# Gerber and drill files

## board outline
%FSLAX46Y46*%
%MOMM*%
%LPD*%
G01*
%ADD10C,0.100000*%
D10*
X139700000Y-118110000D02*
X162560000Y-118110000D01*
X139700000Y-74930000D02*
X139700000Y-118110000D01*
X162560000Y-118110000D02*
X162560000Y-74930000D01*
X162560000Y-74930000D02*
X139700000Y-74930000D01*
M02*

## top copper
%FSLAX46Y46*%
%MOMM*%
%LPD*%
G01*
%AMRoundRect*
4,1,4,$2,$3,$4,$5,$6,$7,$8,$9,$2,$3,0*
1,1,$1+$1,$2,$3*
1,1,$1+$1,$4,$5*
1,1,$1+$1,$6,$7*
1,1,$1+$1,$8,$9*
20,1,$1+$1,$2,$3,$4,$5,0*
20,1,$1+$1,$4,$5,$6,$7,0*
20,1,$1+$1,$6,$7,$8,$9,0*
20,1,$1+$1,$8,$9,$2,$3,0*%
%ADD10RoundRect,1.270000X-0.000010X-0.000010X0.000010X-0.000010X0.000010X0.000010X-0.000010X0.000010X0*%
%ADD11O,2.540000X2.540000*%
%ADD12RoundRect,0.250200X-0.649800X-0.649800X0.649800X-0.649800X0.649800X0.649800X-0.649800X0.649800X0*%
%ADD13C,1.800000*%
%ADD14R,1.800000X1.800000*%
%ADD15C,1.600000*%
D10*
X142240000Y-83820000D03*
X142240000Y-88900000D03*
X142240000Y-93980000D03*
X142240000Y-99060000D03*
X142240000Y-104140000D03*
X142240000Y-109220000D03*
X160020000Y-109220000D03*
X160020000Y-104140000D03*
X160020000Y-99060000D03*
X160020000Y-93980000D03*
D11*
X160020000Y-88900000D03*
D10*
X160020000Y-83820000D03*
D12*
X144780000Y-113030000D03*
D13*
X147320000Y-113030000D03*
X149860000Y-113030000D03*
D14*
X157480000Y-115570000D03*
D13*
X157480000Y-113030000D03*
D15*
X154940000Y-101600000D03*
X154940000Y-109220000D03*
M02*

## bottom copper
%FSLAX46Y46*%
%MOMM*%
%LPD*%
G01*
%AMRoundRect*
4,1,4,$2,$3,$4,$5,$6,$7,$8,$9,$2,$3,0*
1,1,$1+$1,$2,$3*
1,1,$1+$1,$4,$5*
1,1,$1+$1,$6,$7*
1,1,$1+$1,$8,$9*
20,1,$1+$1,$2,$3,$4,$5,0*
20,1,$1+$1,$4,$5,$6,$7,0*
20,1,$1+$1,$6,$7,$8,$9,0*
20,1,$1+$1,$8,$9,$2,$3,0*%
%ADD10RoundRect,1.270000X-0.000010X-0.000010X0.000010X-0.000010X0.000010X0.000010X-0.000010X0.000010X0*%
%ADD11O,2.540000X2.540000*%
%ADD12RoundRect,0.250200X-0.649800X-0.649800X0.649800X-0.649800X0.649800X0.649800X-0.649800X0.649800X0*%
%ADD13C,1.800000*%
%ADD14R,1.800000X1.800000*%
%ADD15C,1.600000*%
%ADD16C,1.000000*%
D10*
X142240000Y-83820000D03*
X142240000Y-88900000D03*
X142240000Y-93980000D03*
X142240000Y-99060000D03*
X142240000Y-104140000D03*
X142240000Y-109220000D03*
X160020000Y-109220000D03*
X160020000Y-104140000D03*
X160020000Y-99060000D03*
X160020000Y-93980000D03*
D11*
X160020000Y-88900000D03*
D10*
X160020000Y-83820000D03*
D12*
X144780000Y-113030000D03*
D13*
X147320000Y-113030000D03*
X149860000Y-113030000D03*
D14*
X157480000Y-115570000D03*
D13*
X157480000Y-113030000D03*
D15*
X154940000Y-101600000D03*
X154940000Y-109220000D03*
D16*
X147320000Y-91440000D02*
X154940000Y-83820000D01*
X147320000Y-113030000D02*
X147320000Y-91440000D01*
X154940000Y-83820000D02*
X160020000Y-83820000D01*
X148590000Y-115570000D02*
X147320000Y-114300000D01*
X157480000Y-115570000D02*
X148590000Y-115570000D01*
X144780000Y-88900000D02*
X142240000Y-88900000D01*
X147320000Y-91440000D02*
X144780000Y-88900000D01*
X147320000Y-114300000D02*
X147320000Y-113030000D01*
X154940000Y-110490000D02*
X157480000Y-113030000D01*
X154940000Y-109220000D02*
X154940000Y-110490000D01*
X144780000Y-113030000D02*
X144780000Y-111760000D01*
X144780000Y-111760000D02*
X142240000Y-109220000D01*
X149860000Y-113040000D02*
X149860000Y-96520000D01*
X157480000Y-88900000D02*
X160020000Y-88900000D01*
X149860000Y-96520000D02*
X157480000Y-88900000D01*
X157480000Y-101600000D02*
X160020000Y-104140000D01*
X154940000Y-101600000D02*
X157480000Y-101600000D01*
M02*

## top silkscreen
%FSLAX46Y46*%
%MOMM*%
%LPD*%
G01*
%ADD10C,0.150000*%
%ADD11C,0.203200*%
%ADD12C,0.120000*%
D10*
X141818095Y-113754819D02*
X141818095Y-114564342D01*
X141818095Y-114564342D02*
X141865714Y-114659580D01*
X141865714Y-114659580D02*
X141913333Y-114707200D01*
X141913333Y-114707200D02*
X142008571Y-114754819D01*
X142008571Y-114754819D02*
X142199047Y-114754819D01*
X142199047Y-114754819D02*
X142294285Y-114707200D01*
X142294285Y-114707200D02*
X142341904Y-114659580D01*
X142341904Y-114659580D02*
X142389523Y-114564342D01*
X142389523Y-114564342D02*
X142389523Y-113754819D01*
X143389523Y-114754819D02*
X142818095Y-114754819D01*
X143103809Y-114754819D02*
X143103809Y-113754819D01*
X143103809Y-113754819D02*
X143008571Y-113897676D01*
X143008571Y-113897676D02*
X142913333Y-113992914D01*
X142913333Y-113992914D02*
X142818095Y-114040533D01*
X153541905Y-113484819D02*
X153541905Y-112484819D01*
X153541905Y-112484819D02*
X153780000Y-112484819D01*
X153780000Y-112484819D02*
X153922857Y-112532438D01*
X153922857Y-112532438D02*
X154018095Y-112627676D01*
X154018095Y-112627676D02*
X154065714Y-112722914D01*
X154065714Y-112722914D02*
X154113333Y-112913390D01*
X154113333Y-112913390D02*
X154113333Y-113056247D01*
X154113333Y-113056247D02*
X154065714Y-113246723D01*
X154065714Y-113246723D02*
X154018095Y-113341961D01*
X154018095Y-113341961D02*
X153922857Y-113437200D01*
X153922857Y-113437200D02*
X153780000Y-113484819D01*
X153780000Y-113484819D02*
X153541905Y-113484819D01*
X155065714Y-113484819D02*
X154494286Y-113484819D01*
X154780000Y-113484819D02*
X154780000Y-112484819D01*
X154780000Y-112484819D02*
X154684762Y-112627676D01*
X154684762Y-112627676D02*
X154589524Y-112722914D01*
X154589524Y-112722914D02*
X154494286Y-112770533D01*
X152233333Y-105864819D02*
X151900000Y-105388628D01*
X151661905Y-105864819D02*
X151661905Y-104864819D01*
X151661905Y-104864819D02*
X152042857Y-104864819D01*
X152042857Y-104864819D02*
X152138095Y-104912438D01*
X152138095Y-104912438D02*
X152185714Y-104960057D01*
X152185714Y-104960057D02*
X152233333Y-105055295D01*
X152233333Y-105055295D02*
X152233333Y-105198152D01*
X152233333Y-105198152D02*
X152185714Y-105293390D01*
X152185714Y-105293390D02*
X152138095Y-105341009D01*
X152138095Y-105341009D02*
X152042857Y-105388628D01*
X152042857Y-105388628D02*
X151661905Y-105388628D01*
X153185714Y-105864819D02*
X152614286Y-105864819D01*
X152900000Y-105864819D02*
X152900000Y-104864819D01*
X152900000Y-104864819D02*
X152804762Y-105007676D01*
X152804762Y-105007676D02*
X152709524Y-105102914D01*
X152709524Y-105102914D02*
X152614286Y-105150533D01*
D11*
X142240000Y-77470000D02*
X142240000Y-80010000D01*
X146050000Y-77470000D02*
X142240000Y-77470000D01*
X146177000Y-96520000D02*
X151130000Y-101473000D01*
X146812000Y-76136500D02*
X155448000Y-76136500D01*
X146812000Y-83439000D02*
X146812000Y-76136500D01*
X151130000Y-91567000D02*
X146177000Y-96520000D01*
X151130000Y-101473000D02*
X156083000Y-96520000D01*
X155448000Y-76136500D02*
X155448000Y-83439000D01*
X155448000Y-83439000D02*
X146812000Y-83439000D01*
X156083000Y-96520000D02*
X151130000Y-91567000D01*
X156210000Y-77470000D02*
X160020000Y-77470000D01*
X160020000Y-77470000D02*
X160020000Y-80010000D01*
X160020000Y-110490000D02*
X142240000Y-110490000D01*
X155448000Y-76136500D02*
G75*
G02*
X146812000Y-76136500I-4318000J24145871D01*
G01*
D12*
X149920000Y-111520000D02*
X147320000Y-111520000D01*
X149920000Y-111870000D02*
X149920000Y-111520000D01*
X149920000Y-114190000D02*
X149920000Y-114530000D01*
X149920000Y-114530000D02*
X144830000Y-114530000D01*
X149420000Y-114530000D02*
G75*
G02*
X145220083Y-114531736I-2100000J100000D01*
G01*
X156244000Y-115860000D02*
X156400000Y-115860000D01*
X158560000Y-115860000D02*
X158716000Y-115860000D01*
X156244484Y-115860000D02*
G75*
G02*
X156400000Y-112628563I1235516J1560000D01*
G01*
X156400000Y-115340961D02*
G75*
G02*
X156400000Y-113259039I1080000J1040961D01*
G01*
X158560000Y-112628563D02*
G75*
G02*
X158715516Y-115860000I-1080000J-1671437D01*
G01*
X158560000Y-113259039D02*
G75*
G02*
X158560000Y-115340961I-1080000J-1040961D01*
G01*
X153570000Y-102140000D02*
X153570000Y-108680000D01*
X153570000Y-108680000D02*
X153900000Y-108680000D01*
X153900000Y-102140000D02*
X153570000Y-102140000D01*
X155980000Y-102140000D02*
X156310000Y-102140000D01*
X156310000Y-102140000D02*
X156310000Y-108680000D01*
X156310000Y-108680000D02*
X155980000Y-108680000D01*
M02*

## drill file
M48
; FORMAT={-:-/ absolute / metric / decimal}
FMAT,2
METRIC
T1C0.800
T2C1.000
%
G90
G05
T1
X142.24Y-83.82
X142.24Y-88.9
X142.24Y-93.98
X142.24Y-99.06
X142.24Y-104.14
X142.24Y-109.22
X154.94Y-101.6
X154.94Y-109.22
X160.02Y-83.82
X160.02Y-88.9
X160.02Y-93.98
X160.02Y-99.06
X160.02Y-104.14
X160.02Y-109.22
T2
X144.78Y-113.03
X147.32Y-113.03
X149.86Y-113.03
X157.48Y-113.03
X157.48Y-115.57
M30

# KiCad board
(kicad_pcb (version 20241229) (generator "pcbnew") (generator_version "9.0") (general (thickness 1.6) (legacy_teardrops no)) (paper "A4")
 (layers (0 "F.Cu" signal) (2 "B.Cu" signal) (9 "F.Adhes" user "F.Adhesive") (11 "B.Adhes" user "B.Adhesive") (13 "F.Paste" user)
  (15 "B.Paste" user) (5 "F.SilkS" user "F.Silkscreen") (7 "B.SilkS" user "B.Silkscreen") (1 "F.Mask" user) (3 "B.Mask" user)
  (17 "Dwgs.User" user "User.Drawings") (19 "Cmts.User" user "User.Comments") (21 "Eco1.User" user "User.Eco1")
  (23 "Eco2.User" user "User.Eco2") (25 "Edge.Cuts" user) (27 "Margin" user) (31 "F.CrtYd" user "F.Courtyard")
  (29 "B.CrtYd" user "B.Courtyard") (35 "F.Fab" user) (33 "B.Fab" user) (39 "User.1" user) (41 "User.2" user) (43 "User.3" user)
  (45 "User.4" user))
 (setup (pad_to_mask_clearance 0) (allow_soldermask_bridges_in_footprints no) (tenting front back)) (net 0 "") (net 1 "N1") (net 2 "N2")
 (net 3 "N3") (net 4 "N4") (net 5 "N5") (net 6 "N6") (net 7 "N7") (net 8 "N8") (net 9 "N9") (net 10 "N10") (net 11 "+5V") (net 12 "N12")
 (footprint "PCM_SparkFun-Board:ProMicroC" (layer "F.Cu") (at 151.13 93.98)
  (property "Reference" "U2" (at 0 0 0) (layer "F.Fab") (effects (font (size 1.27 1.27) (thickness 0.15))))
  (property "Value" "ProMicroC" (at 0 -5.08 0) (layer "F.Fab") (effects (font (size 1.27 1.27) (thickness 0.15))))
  (fp_line (start -8.89 -16.51) (end -8.89 -13.97) (stroke (width 0.2032) (type solid)) (layer "F.SilkS"))
  (fp_line (start -5.08 -16.51) (end -8.89 -16.51) (stroke (width 0.2032) (type solid)) (layer "F.SilkS"))
  (fp_line (start -4.953 2.54) (end 0 7.493) (stroke (width 0.2032) (type solid)) (layer "F.SilkS"))
  (fp_line (start -4.318 -17.8435) (end 4.318 -17.8435) (stroke (width 0.2032) (type solid)) (layer "F.SilkS"))
  (fp_line (start -4.318 -10.541) (end -4.318 -17.8435) (stroke (width 0.2032) (type solid)) (layer "F.SilkS"))
  (fp_line (start 0 -2.413) (end -4.953 2.54) (stroke (width 0.2032) (type solid)) (layer "F.SilkS"))
  (fp_line (start 0 7.493) (end 4.953 2.54) (stroke (width 0.2032) (type solid)) (layer "F.SilkS"))
  (fp_line (start 4.318 -17.8435) (end 4.318 -10.541) (stroke (width 0.2032) (type solid)) (layer "F.SilkS"))
  (fp_line (start 4.318 -10.541) (end -4.318 -10.541) (stroke (width 0.2032) (type solid)) (layer "F.SilkS"))
  (fp_line (start 4.953 2.54) (end 0 -2.413) (stroke (width 0.2032) (type solid)) (layer "F.SilkS"))
  (fp_line (start 5.08 -16.51) (end 8.89 -16.51) (stroke (width 0.2032) (type solid)) (layer "F.SilkS"))
  (fp_line (start 8.89 -16.51) (end 8.89 -13.97) (stroke (width 0.2032) (type solid)) (layer "F.SilkS"))
  (fp_line (start 8.89 16.51) (end -8.89 16.51) (stroke (width 0.2032) (type solid)) (layer "F.SilkS"))
  (fp_arc (start 4.318 -17.8435) (mid 0 -17.460445) (end -4.318 -17.8435) (stroke (width 0.2032) (type solid)) (layer "F.SilkS"))
  (pad "2" thru_hole roundrect (at -8.89 -10.16) (size 2.54 2.54) (drill 0.8) (layers "*.Cu" "*.Mask") (remove_unused_layers no)
   (roundrect_rratio 0.5) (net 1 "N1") (thermal_bridge_angle 0))
  (pad "4" thru_hole roundrect (at -8.89 -5.08) (size 2.54 2.54) (drill 0.8) (layers "*.Cu" "*.Mask") (remove_unused_layers no)
   (roundrect_rratio 0.5) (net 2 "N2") (thermal_bridge_angle 0))
  (pad "6" thru_hole roundrect (at -8.89 0) (size 2.54 2.54) (drill 0.8) (layers "*.Cu" "*.Mask") (remove_unused_layers no)
   (roundrect_rratio 0.5) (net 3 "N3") (thermal_bridge_angle 0))
  (pad "8" thru_hole roundrect (at -8.89 5.08) (size 2.54 2.54) (drill 0.8) (layers "*.Cu" "*.Mask") (remove_unused_layers no)
   (roundrect_rratio 0.5) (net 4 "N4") (thermal_bridge_angle 0))
  (pad "10" thru_hole roundrect (at -8.89 10.16) (size 2.54 2.54) (drill 0.8) (layers "*.Cu" "*.Mask") (remove_unused_layers no)
   (roundrect_rratio 0.5) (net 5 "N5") (thermal_bridge_angle 0))
  (pad "12" thru_hole roundrect (at -8.89 15.24) (size 2.54 2.54) (drill 0.8) (layers "*.Cu" "*.Mask") (remove_unused_layers no)
   (roundrect_rratio 0.5) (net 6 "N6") (thermal_bridge_angle 0))
  (pad "13" thru_hole roundrect (at 8.89 15.24) (size 2.54 2.54) (drill 0.8) (layers "*.Cu" "*.Mask") (remove_unused_layers no)
   (roundrect_rratio 0.5) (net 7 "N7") (thermal_bridge_angle 0))
  (pad "15" thru_hole roundrect (at 8.89 10.16) (size 2.54 2.54) (drill 0.8) (layers "*.Cu" "*.Mask") (remove_unused_layers no)
   (roundrect_rratio 0.5) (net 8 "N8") (thermal_bridge_angle 0))
  (pad "17" thru_hole roundrect (at 8.89 5.08) (size 2.54 2.54) (drill 0.8) (layers "*.Cu" "*.Mask") (remove_unused_layers no)
   (roundrect_rratio 0.5) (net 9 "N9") (thermal_bridge_angle 0))
  (pad "19" thru_hole roundrect (at 8.89 0) (size 2.54 2.54) (drill 0.8) (layers "*.Cu" "*.Mask") (remove_unused_layers no)
   (roundrect_rratio 0.5) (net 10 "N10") (thermal_bridge_angle 0))
  (pad "21" thru_hole oval (at 8.89 -5.08) (size 2.54 2.54) (drill 0.8) (layers "*.Cu" "*.Mask") (remove_unused_layers no) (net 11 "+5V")
   (thermal_bridge_angle 0))
  (pad "23" thru_hole roundrect (at 8.89 -10.16) (size 2.54 2.54) (drill 0.8) (layers "*.Cu" "*.Mask") (remove_unused_layers no)
   (roundrect_rratio 0.5) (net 2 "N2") (thermal_bridge_angle 0)))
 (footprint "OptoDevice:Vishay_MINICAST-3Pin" (layer "F.Cu") (at 144.78 113.03)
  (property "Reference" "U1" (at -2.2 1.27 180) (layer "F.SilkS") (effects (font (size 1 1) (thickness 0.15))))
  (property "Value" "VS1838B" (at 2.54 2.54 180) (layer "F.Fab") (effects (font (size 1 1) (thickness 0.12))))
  (fp_line (start 5.14 -1.51) (end 2.54 -1.51) (stroke (width 0.12) (type solid)) (layer "F.SilkS"))
  (fp_line (start 5.14 -1.16) (end 5.14 -1.51) (stroke (width 0.12) (type solid)) (layer "F.SilkS"))
  (fp_line (start 5.14 1.16) (end 5.14 1.5) (stroke (width 0.12) (type solid)) (layer "F.SilkS"))
  (fp_line (start 5.14 1.5) (end 0.05 1.5) (stroke (width 0.12) (type solid)) (layer "F.SilkS"))
  (fp_arc (start 4.64 1.5) (mid 2.540869 3.502379) (end 0.440083 1.501736) (stroke (width 0.12) (type solid)) (layer "F.SilkS"))
  (pad "1" thru_hole roundrect (at 0 0) (size 1.8 1.8) (drill 1) (layers "*.Cu" "*.Mask") (remove_unused_layers no) (roundrect_rratio 0.139)
   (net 6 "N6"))
  (pad "2" thru_hole circle (at 2.54 0) (size 1.8 1.8) (drill 1) (layers "*.Cu" "*.Mask") (remove_unused_layers no) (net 2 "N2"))
  (pad "3" thru_hole circle (at 5.08 0) (size 1.8 1.8) (drill 1) (layers "*.Cu" "*.Mask") (remove_unused_layers no) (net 11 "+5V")))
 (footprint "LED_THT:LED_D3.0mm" (layer "F.Cu") (at 157.48 115.57 90)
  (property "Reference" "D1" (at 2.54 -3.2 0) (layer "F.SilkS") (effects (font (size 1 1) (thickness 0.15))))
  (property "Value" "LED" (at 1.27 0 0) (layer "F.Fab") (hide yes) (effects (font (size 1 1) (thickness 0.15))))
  (fp_line (start -0.29 -1.236) (end -0.29 -1.08) (stroke (width 0.12) (type solid)) (layer "F.SilkS"))
  (fp_line (start -0.29 1.08) (end -0.29 1.236) (stroke (width 0.12) (type solid)) (layer "F.SilkS"))
  (fp_arc (start -0.29 -1.235516) (mid 1.36566 -1.987699) (end 2.941437 -1.08) (stroke (width 0.12) (type solid)) (layer "F.SilkS"))
  (fp_arc (start 0.229039 -1.08) (mid 1.27 -1.5) (end 2.310961 -1.08) (stroke (width 0.12) (type solid)) (layer "F.SilkS"))
  (fp_arc (start 2.941437 1.08) (mid 1.36566 1.987699) (end -0.29 1.235516) (stroke (width 0.12) (type solid)) (layer "F.SilkS"))
  (fp_arc (start 2.310961 1.08) (mid 1.27 1.5) (end 0.229039 1.08) (stroke (width 0.12) (type solid)) (layer "F.SilkS"))
  (pad "1" thru_hole rect (at 0 0 90) (size 1.8 1.8) (drill 1) (layers "*.Cu" "*.Mask") (remove_unused_layers no) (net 2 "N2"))
  (pad "2" thru_hole circle (at 2.54 0 90) (size 1.8 1.8) (drill 1) (layers "*.Cu" "*.Mask") (remove_unused_layers no) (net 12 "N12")))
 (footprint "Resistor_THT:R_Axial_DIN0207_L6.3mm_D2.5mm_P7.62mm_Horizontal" (layer "F.Cu") (at 154.94 101.6 -90)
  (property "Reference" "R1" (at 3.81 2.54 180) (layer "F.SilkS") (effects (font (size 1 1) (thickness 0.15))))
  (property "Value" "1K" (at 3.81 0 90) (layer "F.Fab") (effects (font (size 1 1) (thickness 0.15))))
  (fp_line (start 0.54 1.37) (end 7.08 1.37) (stroke (width 0.12) (type solid)) (layer "F.SilkS"))
  (fp_line (start 7.08 1.37) (end 7.08 1.04) (stroke (width 0.12) (type solid)) (layer "F.SilkS"))
  (fp_line (start 0.54 1.04) (end 0.54 1.37) (stroke (width 0.12) (type solid)) (layer "F.SilkS"))
  (fp_line (start 0.54 -1.04) (end 0.54 -1.37) (stroke (width 0.12) (type solid)) (layer "F.SilkS"))
  (fp_line (start 0.54 -1.37) (end 7.08 -1.37) (stroke (width 0.12) (type solid)) (layer "F.SilkS"))
  (fp_line (start 7.08 -1.37) (end 7.08 -1.04) (stroke (width 0.12) (type solid)) (layer "F.SilkS"))
  (pad "1" thru_hole circle (at 0 0 270) (size 1.6 1.6) (drill 0.8) (layers "*.Cu" "*.Mask") (remove_unused_layers no) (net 8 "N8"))
  (pad "2" thru_hole circle (at 7.62 0 270) (size 1.6 1.6) (drill 0.8) (layers "*.Cu" "*.Mask") (remove_unused_layers no) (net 12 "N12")))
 (gr_line (start 139.7 118.11) (end 162.56 118.11) (stroke (width 0.1) (type solid)) (layer "Edge.Cuts"))
 (gr_line (start 139.7 74.93) (end 139.7 118.11) (stroke (width 0.1) (type default)) (layer "Edge.Cuts"))
 (gr_line (start 162.56 118.11) (end 162.56 74.93) (stroke (width 0.1) (type default)) (layer "Edge.Cuts"))
 (gr_line (start 162.56 74.93) (end 139.7 74.93) (stroke (width 0.1) (type solid)) (layer "Edge.Cuts"))
 (segment (start 147.32 91.44) (end 154.94 83.82) (width 1) (layer "B.Cu") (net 2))
 (segment (start 147.32 113.03) (end 147.32 91.44) (width 1) (layer "B.Cu") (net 2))
 (segment (start 154.94 83.82) (end 160.02 83.82) (width 1) (layer "B.Cu") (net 2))
 (segment (start 148.59 115.57) (end 147.32 114.3) (width 1) (layer "B.Cu") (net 2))
 (segment (start 157.48 115.57) (end 148.59 115.57) (width 1) (layer "B.Cu") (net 2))
 (segment (start 144.78 88.9) (end 142.24 88.9) (width 1) (layer "B.Cu") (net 2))
 (segment (start 147.32 91.44) (end 144.78 88.9) (width 1) (layer "B.Cu") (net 2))
 (segment (start 147.32 114.3) (end 147.32 113.03) (width 1) (layer "B.Cu") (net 2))
 (segment (start 154.94 110.49) (end 157.48 113.03) (width 1) (layer "B.Cu") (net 12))
 (segment (start 154.94 109.22) (end 154.94 110.49) (width 1) (layer "B.Cu") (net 12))
 (segment (start 144.78 113.03) (end 144.78 111.76) (width 1) (layer "B.Cu") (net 6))
 (segment (start 144.78 111.76) (end 142.24 109.22) (width 1) (layer "B.Cu") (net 6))
 (segment (start 149.86 113.04) (end 149.86 96.52) (width 1) (layer "B.Cu") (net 11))
 (segment (start 157.48 88.9) (end 160.02 88.9) (width 1) (layer "B.Cu") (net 11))
 (segment (start 149.86 96.52) (end 157.48 88.9) (width 1) (layer "B.Cu") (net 11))
 (segment (start 157.48 101.6) (end 160.02 104.14) (width 1) (layer "B.Cu") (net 8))
 (segment (start 154.94 101.6) (end 157.48 101.6) (width 1) (layer "B.Cu") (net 8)))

